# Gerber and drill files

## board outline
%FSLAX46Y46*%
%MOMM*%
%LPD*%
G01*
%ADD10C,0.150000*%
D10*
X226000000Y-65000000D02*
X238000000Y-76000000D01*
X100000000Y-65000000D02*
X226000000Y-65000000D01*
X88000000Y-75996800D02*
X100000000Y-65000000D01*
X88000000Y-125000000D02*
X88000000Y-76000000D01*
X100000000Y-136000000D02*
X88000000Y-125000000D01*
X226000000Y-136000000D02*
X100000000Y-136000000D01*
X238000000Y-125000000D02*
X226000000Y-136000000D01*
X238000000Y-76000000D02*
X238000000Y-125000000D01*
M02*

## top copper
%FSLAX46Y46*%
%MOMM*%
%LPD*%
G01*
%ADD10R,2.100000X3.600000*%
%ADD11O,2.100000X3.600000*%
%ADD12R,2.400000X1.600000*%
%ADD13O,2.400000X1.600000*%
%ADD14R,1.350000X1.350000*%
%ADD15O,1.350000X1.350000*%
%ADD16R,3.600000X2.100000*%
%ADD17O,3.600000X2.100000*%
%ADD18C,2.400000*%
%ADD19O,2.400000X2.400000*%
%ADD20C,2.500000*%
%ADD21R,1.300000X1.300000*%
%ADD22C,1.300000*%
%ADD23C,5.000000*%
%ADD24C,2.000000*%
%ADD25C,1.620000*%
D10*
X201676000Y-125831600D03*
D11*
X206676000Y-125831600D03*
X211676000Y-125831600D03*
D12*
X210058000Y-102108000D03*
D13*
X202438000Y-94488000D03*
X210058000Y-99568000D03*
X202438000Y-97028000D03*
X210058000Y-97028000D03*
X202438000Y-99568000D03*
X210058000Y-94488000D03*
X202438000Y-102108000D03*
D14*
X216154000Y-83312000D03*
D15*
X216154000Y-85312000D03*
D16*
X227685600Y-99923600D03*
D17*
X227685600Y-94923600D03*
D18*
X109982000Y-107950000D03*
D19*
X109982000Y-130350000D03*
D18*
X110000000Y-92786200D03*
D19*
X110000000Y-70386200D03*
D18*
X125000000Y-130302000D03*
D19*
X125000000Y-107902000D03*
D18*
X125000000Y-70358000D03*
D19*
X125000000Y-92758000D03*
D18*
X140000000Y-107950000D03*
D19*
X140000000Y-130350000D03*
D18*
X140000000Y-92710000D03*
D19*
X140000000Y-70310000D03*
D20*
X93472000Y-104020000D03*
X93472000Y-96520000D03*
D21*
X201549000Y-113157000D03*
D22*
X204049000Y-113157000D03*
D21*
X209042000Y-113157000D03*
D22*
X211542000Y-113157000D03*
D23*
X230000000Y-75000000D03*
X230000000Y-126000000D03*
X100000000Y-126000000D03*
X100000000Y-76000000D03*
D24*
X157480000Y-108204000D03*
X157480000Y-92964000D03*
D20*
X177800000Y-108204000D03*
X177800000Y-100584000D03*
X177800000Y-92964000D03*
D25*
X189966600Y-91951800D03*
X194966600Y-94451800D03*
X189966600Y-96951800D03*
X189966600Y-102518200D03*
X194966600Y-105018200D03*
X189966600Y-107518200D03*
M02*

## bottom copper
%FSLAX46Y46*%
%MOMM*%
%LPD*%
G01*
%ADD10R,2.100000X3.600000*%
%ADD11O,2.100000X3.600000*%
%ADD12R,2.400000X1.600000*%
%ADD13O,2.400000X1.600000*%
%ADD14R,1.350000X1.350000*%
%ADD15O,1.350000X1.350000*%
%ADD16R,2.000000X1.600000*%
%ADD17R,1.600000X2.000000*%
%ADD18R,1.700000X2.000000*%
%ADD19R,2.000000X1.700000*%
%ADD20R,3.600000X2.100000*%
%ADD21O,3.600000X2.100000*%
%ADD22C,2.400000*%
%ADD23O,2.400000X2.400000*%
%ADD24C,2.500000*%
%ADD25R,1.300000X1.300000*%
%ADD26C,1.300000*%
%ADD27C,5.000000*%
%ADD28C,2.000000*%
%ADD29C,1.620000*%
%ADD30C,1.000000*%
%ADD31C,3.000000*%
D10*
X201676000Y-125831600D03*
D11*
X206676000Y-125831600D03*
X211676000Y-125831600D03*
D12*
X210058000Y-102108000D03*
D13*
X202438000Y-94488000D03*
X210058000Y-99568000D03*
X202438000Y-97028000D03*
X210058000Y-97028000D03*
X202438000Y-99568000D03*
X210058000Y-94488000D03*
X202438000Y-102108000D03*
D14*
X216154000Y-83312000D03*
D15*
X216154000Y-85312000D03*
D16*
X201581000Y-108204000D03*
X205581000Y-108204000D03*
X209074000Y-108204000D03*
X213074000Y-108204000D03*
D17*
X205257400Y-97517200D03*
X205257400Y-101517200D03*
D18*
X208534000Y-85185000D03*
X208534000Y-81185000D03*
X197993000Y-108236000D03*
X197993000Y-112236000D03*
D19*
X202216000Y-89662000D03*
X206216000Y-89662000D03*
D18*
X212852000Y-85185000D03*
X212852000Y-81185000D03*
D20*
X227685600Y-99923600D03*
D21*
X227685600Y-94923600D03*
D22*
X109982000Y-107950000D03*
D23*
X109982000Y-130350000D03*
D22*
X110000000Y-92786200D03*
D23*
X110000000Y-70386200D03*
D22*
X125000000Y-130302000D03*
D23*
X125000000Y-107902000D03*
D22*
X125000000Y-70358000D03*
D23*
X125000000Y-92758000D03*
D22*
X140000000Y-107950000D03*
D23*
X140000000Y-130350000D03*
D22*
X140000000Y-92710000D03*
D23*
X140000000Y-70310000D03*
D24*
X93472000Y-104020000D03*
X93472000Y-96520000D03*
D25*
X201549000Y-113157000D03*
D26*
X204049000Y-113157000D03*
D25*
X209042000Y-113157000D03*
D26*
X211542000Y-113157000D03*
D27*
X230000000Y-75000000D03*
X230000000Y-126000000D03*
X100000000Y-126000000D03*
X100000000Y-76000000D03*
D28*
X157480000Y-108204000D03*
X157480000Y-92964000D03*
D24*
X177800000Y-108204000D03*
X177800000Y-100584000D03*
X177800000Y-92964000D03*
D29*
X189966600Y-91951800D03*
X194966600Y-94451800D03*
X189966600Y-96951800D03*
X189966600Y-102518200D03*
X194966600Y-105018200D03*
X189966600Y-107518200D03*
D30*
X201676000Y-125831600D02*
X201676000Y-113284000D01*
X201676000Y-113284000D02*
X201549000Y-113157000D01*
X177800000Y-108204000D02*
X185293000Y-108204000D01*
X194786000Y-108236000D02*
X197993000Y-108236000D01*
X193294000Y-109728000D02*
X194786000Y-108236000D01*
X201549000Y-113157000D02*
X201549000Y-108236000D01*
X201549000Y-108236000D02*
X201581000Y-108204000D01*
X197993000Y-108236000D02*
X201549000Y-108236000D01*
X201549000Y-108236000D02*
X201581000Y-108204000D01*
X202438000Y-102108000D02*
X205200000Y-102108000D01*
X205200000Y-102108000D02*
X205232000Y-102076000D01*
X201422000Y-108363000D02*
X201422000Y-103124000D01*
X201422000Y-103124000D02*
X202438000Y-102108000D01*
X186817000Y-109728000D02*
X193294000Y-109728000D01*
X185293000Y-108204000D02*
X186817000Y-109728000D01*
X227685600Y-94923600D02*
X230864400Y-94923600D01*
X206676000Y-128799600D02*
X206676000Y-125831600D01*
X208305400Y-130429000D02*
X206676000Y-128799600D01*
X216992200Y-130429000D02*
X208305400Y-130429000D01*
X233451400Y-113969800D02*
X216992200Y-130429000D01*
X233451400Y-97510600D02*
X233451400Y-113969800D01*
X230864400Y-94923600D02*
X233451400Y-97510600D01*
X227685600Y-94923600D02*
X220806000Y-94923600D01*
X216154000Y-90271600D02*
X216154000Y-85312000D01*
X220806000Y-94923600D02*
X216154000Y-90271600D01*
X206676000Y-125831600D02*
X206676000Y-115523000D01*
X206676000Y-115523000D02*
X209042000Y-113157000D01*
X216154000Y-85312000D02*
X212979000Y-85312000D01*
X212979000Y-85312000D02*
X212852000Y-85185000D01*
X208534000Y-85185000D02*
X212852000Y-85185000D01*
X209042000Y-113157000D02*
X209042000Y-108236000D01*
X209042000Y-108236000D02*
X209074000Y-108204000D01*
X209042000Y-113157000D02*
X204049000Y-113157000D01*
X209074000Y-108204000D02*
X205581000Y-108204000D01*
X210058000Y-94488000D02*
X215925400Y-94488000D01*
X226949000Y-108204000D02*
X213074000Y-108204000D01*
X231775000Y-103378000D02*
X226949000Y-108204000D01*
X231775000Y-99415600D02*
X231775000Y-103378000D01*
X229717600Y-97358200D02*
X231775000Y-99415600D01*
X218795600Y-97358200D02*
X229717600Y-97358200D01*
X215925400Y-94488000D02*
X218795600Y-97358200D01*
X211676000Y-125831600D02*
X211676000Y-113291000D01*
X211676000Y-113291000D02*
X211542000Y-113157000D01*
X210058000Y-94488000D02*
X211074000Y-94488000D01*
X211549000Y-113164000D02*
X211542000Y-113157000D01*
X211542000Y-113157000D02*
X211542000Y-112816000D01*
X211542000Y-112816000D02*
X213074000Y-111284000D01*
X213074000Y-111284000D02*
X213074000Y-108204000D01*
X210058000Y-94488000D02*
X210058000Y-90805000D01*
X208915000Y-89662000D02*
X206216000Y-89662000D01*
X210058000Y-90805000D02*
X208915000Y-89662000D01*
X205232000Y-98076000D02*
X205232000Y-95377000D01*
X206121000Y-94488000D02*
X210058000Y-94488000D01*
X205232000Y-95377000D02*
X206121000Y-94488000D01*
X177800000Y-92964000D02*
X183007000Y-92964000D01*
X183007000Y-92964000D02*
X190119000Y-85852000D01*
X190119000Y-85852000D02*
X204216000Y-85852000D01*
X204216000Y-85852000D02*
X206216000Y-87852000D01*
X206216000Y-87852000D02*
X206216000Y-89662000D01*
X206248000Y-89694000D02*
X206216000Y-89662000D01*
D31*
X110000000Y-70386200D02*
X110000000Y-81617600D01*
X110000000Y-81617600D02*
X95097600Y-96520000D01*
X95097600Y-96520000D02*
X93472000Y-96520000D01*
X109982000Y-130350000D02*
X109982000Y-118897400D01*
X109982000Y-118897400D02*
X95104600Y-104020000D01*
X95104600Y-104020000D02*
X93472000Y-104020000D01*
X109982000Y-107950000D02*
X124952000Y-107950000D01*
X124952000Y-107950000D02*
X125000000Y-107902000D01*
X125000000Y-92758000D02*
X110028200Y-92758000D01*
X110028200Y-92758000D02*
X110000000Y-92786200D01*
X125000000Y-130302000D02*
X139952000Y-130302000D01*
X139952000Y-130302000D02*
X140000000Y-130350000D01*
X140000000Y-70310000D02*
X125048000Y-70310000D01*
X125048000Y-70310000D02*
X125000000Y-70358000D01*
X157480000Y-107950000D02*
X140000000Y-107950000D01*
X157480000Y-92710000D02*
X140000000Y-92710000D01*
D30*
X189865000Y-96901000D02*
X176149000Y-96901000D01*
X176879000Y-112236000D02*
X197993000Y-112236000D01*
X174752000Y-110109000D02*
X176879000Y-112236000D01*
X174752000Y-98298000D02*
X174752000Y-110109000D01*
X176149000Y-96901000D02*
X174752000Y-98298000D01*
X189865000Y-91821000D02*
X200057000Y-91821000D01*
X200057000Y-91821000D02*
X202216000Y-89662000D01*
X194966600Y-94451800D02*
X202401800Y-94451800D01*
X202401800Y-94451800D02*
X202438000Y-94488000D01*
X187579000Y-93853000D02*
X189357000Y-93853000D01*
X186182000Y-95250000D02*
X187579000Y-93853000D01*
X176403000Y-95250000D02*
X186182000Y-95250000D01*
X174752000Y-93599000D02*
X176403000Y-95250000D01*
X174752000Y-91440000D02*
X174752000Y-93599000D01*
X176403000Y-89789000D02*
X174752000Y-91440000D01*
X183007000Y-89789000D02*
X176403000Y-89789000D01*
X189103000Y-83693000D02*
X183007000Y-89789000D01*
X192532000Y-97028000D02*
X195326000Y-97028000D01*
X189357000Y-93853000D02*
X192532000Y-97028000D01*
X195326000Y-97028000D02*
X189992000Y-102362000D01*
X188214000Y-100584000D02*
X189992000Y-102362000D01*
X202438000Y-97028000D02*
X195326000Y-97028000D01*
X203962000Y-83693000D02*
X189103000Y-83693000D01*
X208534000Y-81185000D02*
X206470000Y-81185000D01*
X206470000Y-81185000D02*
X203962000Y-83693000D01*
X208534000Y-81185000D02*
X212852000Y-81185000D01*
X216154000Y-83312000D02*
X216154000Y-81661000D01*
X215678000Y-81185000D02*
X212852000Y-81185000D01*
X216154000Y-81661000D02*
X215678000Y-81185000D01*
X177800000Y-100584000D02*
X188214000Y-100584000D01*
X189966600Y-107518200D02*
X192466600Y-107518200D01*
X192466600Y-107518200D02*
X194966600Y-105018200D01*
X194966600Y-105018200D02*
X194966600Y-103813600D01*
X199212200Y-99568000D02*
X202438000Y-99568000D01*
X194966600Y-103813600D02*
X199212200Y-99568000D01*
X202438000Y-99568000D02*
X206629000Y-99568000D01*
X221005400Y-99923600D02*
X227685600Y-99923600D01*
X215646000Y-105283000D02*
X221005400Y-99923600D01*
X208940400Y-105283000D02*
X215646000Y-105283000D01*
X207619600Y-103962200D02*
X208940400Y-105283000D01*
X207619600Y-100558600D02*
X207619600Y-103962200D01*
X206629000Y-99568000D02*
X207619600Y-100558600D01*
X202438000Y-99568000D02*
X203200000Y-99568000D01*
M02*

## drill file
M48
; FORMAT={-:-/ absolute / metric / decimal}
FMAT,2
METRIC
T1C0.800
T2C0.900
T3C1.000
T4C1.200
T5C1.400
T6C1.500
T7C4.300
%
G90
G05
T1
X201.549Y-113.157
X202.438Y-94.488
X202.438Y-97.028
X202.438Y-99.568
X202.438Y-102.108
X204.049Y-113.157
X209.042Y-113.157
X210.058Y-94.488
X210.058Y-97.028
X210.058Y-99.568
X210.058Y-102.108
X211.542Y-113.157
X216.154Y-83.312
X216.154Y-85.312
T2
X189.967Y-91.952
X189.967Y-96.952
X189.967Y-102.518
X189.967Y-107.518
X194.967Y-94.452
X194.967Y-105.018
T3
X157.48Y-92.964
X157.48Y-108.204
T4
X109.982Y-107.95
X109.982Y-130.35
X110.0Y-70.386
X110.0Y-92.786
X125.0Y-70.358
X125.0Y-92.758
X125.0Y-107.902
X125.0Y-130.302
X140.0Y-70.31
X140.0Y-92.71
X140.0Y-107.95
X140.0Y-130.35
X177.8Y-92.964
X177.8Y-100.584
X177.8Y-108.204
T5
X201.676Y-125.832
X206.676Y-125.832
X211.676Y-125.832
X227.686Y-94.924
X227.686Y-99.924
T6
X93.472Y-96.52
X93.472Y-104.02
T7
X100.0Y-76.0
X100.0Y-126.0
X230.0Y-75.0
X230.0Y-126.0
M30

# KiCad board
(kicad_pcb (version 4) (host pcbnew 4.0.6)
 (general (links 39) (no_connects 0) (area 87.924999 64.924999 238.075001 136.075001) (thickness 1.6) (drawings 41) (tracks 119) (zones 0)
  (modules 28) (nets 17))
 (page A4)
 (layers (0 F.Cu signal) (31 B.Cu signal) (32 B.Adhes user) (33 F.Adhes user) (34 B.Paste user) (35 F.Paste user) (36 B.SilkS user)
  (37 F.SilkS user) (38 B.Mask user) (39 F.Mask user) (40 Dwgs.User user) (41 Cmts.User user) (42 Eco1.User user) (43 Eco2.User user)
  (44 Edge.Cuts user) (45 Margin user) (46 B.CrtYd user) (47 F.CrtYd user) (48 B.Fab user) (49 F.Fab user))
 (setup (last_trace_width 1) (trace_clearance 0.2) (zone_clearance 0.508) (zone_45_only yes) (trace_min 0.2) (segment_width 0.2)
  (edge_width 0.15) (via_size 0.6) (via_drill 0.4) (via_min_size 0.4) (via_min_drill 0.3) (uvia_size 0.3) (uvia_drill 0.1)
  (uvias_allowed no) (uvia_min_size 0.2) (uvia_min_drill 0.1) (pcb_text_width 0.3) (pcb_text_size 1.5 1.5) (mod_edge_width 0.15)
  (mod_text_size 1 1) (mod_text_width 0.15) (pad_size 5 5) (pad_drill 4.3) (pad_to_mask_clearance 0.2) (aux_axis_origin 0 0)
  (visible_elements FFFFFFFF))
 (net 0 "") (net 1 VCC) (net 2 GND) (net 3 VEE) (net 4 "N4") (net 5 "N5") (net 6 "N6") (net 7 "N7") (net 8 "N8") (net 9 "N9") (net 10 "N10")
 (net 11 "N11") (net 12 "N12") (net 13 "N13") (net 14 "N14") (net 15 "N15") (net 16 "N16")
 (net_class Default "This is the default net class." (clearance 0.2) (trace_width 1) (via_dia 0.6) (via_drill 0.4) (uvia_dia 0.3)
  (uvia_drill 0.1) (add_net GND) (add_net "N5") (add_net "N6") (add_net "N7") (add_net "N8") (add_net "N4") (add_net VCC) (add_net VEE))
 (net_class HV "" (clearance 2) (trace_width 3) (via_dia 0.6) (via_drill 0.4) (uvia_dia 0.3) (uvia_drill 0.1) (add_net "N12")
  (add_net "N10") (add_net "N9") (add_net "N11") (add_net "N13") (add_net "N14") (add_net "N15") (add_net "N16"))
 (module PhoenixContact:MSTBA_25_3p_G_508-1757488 (layer F.Cu) (at 201.676 125.8316)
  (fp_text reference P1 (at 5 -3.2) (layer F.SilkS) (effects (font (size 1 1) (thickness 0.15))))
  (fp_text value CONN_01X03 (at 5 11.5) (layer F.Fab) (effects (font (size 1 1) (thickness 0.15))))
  (pad 1 thru_hole rect (at 0 0) (size 2.1 3.6) (drill 1.4) (layers *.Cu *.Mask) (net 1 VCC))
  (pad 2 thru_hole oval (at 5 0) (size 2.1 3.6) (drill 1.4) (layers *.Cu *.Mask) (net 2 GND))
  (pad 3 thru_hole oval (at 10 0) (size 2.1 3.6) (drill 1.4) (layers *.Cu *.Mask) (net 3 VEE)))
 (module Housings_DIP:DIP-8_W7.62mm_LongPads (layer F.Cu) (at 210.058 102.108 180)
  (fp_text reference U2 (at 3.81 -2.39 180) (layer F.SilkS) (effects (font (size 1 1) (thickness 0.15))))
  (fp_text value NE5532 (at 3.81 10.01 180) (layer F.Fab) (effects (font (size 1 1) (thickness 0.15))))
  (pad 1 thru_hole rect (at 0 0 180) (size 2.4 1.6) (drill 0.8) (layers *.Cu *.Mask))
  (pad 5 thru_hole oval (at 7.62 7.62 180) (size 2.4 1.6) (drill 0.8) (layers *.Cu *.Mask) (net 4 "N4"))
  (pad 2 thru_hole oval (at 0 2.54 180) (size 2.4 1.6) (drill 0.8) (layers *.Cu *.Mask))
  (pad 6 thru_hole oval (at 7.62 5.08 180) (size 2.4 1.6) (drill 0.8) (layers *.Cu *.Mask) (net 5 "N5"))
  (pad 3 thru_hole oval (at 0 5.08 180) (size 2.4 1.6) (drill 0.8) (layers *.Cu *.Mask))
  (pad 7 thru_hole oval (at 7.62 2.54 180) (size 2.4 1.6) (drill 0.8) (layers *.Cu *.Mask) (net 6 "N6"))
  (pad 4 thru_hole oval (at 0 7.62 180) (size 2.4 1.6) (drill 0.8) (layers *.Cu *.Mask) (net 3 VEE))
  (pad 8 thru_hole oval (at 7.62 0 180) (size 2.4 1.6) (drill 0.8) (layers *.Cu *.Mask) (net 1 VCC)))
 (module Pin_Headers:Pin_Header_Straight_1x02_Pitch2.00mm (layer F.Cu) (at 216.154 83.312)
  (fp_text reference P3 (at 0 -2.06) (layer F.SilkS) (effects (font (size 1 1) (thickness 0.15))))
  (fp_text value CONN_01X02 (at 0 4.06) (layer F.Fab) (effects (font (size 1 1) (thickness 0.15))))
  (pad 1 thru_hole rect (at 0 0) (size 1.35 1.35) (drill 0.8) (layers *.Cu *.Mask) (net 5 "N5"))
  (pad 2 thru_hole oval (at 0 2) (size 1.35 1.35) (drill 0.8) (layers *.Cu *.Mask) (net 2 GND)))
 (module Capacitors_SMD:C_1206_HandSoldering (layer B.Cu) (at 203.581 108.204)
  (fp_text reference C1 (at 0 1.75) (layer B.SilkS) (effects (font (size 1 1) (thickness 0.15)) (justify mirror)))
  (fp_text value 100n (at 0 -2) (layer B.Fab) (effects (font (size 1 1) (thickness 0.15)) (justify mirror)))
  (pad 1 smd rect (at -2 0) (size 2 1.6) (layers B.Cu B.Paste B.Mask) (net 1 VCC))
  (pad 2 smd rect (at 2 0) (size 2 1.6) (layers B.Cu B.Paste B.Mask) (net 2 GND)))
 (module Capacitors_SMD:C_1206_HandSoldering (layer B.Cu) (at 211.074 108.204)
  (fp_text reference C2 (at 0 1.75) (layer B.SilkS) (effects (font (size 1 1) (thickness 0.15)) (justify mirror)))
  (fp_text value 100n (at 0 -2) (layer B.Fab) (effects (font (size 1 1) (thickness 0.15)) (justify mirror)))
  (pad 1 smd rect (at -2 0) (size 2 1.6) (layers B.Cu B.Paste B.Mask) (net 2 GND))
  (pad 2 smd rect (at 2 0) (size 2 1.6) (layers B.Cu B.Paste B.Mask) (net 3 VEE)))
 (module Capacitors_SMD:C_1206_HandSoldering (layer B.Cu) (at 205.2574 99.5172 270)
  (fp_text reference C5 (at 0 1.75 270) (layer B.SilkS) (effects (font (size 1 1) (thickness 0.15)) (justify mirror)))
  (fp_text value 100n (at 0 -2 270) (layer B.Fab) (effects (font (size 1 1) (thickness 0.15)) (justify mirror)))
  (pad 1 smd rect (at -2 0 270) (size 2 1.6) (layers B.Cu B.Paste B.Mask) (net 3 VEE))
  (pad 2 smd rect (at 2 0 270) (size 2 1.6) (layers B.Cu B.Paste B.Mask) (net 1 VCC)))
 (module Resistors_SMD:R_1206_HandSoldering (layer B.Cu) (at 208.534 83.185 90)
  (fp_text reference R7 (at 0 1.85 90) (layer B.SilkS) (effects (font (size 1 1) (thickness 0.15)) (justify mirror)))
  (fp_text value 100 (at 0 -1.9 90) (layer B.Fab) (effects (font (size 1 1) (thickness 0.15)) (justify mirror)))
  (pad 1 smd rect (at -2 0 90) (size 2 1.7) (layers B.Cu B.Paste B.Mask) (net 2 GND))
  (pad 2 smd rect (at 2 0 90) (size 2 1.7) (layers B.Cu B.Paste B.Mask) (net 5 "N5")))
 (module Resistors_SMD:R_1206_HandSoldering (layer B.Cu) (at 197.993 110.236 270)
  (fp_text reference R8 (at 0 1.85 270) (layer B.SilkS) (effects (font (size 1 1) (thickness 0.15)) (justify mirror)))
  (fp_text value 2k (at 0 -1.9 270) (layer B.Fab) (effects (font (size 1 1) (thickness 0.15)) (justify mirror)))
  (pad 1 smd rect (at -2 0 270) (size 2 1.7) (layers B.Cu B.Paste B.Mask) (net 1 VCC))
  (pad 2 smd rect (at 2 0 270) (size 2 1.7) (layers B.Cu B.Paste B.Mask) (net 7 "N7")))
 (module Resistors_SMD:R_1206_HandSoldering (layer B.Cu) (at 204.216 89.662)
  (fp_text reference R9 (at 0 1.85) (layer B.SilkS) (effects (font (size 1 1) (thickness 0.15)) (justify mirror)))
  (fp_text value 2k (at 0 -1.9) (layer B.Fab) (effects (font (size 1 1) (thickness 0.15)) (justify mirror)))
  (pad 1 smd rect (at -2 0) (size 2 1.7) (layers B.Cu B.Paste B.Mask) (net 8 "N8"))
  (pad 2 smd rect (at 2 0) (size 2 1.7) (layers B.Cu B.Paste B.Mask) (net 3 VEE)))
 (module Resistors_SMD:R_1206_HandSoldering (layer B.Cu) (at 212.852 83.185 90)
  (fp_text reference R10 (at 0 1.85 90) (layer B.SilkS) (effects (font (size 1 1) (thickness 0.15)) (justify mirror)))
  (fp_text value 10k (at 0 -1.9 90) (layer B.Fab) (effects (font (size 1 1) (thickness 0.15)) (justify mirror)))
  (pad 1 smd rect (at -2 0 90) (size 2 1.7) (layers B.Cu B.Paste B.Mask) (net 2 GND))
  (pad 2 smd rect (at 2 0 90) (size 2 1.7) (layers B.Cu B.Paste B.Mask) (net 5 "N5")))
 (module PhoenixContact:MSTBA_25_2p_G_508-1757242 (layer F.Cu) (at 227.6856 99.9236 90)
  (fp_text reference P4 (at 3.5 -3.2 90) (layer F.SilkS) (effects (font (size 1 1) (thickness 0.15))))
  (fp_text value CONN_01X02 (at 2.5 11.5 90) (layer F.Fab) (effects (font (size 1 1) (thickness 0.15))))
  (pad 1 thru_hole rect (at 0 0 90) (size 2.1 3.6) (drill 1.4) (layers *.Cu *.Mask) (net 6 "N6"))
  (pad 2 thru_hole oval (at 5 0 90) (size 2.1 3.6) (drill 1.4) (layers *.Cu *.Mask) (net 2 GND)))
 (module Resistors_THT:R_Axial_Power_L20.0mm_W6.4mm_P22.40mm (layer F.Cu) (at 109.982 107.95 270)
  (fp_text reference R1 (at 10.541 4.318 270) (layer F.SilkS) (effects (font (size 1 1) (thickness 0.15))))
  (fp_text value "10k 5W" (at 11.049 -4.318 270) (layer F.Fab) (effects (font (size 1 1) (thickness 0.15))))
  (pad 1 thru_hole circle (at 0 0 270) (size 2.4 2.4) (drill 1.2) (layers *.Cu *.Mask) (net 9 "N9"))
  (pad 2 thru_hole oval (at 22.4 0 270) (size 2.4 2.4) (drill 1.2) (layers *.Cu *.Mask) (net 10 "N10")))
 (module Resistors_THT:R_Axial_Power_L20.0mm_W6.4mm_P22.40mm (layer F.Cu) (at 110 92.7862 90)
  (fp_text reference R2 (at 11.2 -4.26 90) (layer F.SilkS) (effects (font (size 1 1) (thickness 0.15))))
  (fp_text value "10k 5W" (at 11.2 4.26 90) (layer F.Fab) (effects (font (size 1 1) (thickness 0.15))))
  (pad 1 thru_hole circle (at 0 0 90) (size 2.4 2.4) (drill 1.2) (layers *.Cu *.Mask) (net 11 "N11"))
  (pad 2 thru_hole oval (at 22.4 0 90) (size 2.4 2.4) (drill 1.2) (layers *.Cu *.Mask) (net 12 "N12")))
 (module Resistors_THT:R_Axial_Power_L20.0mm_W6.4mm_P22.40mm (layer F.Cu) (at 125 130.302 90)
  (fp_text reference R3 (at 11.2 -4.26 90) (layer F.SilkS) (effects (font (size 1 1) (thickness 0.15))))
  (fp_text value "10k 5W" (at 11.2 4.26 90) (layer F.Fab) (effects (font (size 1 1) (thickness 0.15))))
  (pad 1 thru_hole circle (at 0 0 90) (size 2.4 2.4) (drill 1.2) (layers *.Cu *.Mask) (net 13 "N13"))
  (pad 2 thru_hole oval (at 22.4 0 90) (size 2.4 2.4) (drill 1.2) (layers *.Cu *.Mask) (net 9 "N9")))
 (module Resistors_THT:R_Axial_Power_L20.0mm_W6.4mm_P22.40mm (layer F.Cu) (at 125 70.358 270)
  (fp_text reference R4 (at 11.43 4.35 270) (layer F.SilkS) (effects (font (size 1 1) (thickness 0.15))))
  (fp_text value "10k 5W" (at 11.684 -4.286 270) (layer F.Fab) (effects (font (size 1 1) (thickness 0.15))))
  (pad 1 thru_hole circle (at 0 0 270) (size 2.4 2.4) (drill 1.2) (layers *.Cu *.Mask) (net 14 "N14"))
  (pad 2 thru_hole oval (at 22.4 0 270) (size 2.4 2.4) (drill 1.2) (layers *.Cu *.Mask) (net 11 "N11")))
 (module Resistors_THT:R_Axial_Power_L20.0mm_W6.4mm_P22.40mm (layer F.Cu) (at 140 107.95 270)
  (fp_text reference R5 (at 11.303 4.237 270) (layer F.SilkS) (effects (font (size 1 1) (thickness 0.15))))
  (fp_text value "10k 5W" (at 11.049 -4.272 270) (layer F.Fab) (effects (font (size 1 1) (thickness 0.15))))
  (pad 1 thru_hole circle (at 0 0 270) (size 2.4 2.4) (drill 1.2) (layers *.Cu *.Mask) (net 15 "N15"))
  (pad 2 thru_hole oval (at 22.4 0 270) (size 2.4 2.4) (drill 1.2) (layers *.Cu *.Mask) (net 13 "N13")))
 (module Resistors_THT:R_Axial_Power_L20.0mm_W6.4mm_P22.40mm (layer F.Cu) (at 140 92.71 90)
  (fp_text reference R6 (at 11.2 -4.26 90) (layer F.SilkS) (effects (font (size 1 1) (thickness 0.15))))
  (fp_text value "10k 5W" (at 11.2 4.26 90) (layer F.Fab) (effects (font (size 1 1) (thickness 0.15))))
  (pad 1 thru_hole circle (at 0 0 90) (size 2.4 2.4) (drill 1.2) (layers *.Cu *.Mask) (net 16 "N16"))
  (pad 2 thru_hole oval (at 22.4 0 90) (size 2.4 2.4) (drill 1.2) (layers *.Cu *.Mask) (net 14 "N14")))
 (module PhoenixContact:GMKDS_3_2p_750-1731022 (layer F.Cu) (at 93.472 96.52 270)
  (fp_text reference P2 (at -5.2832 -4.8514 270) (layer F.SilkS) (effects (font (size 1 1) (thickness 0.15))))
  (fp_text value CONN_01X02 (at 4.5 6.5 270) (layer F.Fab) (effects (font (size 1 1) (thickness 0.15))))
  (pad 2 thru_hole circle (at 7.5 0 270) (size 2.5 2.5) (drill 1.5) (layers *.Cu *.Mask) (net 10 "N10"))
  (pad 1 thru_hole circle (at 0 0 270) (size 2.5 2.5) (drill 1.5) (layers *.Cu *.Mask) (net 12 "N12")))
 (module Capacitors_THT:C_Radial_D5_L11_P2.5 (layer F.Cu) (at 201.549 113.157)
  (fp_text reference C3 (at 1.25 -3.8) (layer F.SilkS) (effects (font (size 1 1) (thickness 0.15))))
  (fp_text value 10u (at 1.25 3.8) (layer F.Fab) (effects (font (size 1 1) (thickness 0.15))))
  (pad 1 thru_hole rect (at 0 0) (size 1.3 1.3) (drill 0.8) (layers *.Cu *.Mask) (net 1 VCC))
  (pad 2 thru_hole circle (at 2.5 0) (size 1.3 1.3) (drill 0.8) (layers *.Cu *.Mask) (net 2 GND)))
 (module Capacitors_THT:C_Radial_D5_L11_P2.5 (layer F.Cu) (at 209.042 113.157)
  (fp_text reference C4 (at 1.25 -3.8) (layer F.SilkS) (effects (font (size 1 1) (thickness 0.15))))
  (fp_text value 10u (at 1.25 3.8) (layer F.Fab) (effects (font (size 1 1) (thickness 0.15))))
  (pad 1 thru_hole rect (at 0 0) (size 1.3 1.3) (drill 0.8) (layers *.Cu *.Mask) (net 2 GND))
  (pad 2 thru_hole circle (at 2.5 0) (size 1.3 1.3) (drill 0.8) (layers *.Cu *.Mask) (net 3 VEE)))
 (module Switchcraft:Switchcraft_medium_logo (layer F.Cu) (at 208.7372 69.3166)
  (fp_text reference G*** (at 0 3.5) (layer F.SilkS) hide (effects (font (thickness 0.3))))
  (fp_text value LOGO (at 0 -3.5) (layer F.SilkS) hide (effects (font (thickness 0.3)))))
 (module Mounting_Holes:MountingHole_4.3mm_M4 (layer F.Cu) (at 230 75)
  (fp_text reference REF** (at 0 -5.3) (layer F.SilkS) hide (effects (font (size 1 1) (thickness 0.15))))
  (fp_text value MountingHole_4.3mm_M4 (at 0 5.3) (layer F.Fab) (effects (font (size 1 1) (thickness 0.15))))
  (pad "" np_thru_hole circle (at 0 0) (size 5 5) (drill 4.3) (layers *.Cu *.Mask)))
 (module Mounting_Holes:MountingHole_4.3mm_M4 (layer F.Cu) (at 230 126)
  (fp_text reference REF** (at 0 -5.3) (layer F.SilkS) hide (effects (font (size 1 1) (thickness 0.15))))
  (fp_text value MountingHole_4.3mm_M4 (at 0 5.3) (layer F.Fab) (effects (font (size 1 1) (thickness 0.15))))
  (pad "" np_thru_hole circle (at 0 0) (size 5 5) (drill 4.3) (layers *.Cu *.Mask)))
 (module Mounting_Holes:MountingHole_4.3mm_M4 (layer F.Cu) (at 100 126)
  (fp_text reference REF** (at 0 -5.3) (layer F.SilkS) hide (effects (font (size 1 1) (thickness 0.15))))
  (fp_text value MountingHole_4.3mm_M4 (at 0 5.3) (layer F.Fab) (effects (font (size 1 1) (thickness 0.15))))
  (pad "" np_thru_hole circle (at 0 0) (size 5 5) (drill 4.3) (layers *.Cu *.Mask)))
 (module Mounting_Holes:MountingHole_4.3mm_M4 (layer F.Cu) (at 100 76)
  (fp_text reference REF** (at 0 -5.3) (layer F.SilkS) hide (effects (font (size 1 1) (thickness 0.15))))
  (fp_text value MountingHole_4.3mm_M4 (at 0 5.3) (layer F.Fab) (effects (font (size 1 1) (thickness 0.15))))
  (pad "" np_thru_hole circle (at 0 0) (size 5 5) (drill 4.3) (layers *.Cu *.Mask)))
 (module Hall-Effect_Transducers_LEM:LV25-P (layer F.Cu) (at 167.64 100.584 90)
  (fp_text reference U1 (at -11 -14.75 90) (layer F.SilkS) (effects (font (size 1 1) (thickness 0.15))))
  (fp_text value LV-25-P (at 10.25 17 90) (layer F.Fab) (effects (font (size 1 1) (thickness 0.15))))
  (pad 1 thru_hole circle (at -7.62 -10.16 90) (size 2 2) (drill 1) (layers *.Cu *.Mask) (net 15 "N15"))
  (pad 2 thru_hole circle (at 7.62 -10.16 90) (size 2 2) (drill 1) (layers *.Cu *.Mask) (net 16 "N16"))
  (pad 3 thru_hole circle (at -7.62 10.16 90) (size 2.5 2.5) (drill 1.2) (layers *.Cu *.Mask) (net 1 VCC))
  (pad 4 thru_hole circle (at 0 10.16 90) (size 2.5 2.5) (drill 1.2) (layers *.Cu *.Mask) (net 5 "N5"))
  (pad 5 thru_hole circle (at 7.62 10.16 90) (size 2.5 2.5) (drill 1.2) (layers *.Cu *.Mask) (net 3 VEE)))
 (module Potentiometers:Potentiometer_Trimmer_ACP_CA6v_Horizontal (layer F.Cu) (at 189.9666 96.9518)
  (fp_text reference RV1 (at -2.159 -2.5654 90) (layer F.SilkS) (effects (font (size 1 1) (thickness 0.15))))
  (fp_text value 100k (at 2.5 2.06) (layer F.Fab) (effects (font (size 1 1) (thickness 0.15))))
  (pad 3 thru_hole circle (at 0 -5) (size 1.62 1.62) (drill 0.9) (layers *.Cu *.Mask) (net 8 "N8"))
  (pad 2 thru_hole circle (at 5 -2.5) (size 1.62 1.62) (drill 0.9) (layers *.Cu *.Mask) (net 4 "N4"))
  (pad 1 thru_hole circle (at 0 0) (size 1.62 1.62) (drill 0.9) (layers *.Cu *.Mask) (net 7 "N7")))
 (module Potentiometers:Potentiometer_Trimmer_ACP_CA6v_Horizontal (layer F.Cu) (at 189.9666 107.5182)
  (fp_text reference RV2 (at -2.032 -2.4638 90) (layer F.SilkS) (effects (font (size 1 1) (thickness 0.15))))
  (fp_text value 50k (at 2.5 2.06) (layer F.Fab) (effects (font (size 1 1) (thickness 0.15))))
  (pad 3 thru_hole circle (at 0 -5) (size 1.62 1.62) (drill 0.9) (layers *.Cu *.Mask) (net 5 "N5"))
  (pad 2 thru_hole circle (at 5 -2.5) (size 1.62 1.62) (drill 0.9) (layers *.Cu *.Mask) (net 6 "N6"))
  (pad 1 thru_hole circle (at 0 0) (size 1.62 1.62) (drill 0.9) (layers *.Cu *.Mask) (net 6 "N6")))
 (gr_line (start 226 65) (end 238 76) (angle 90) (layer Edge.Cuts) (width 0.15))
 (gr_line (start 100 65) (end 226 65) (angle 90) (layer Edge.Cuts) (width 0.15))
 (gr_line (start 88 75.9968) (end 100 65) (angle 90) (layer Edge.Cuts) (width 0.15))
 (gr_line (start 88 125) (end 88 76) (angle 90) (layer Edge.Cuts) (width 0.15))
 (gr_line (start 100 136) (end 88 125) (angle 90) (layer Edge.Cuts) (width 0.15))
 (gr_line (start 226 136) (end 100 136) (angle 90) (layer Edge.Cuts) (width 0.15))
 (gr_line (start 238 125) (end 226 136) (angle 90) (layer Edge.Cuts) (width 0.15))
 (gr_line (start 238 76) (end 238 125) (angle 90) (layer Edge.Cuts) (width 0.15))
 (segment (start 201.676 125.8316) (end 201.676 113.284) (width 1) (layer B.Cu) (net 1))
 (segment (start 201.676 113.284) (end 201.549 113.157) (width 1) (layer B.Cu) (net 1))
 (segment (start 177.8 108.204) (end 185.293 108.204) (width 1) (layer B.Cu) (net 1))
 (segment (start 194.786 108.236) (end 197.993 108.236) (width 1) (layer B.Cu) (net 1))
 (segment (start 193.294 109.728) (end 194.786 108.236) (width 1) (layer B.Cu) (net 1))
 (segment (start 201.549 113.157) (end 201.549 108.236) (width 1) (layer B.Cu) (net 1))
 (segment (start 201.549 108.236) (end 201.581 108.204) (width 1) (layer B.Cu) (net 1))
 (segment (start 197.993 108.236) (end 201.549 108.236) (width 1) (layer B.Cu) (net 1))
 (segment (start 201.549 108.236) (end 201.581 108.204) (width 1) (layer B.Cu) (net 1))
 (segment (start 202.438 102.108) (end 205.2 102.108) (width 1) (layer B.Cu) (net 1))
 (segment (start 205.2 102.108) (end 205.232 102.076) (width 1) (layer B.Cu) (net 1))
 (segment (start 201.422 108.363) (end 201.422 103.124) (width 1) (layer B.Cu) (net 1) (status 10))
 (segment (start 201.422 103.124) (end 202.438 102.108) (width 1) (layer B.Cu) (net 1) (status 20))
 (segment (start 186.817 109.728) (end 193.294 109.728) (width 1) (layer B.Cu) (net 1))
 (segment (start 185.293 108.204) (end 186.817 109.728) (width 1) (layer B.Cu) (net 1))
 (segment (start 227.6856 94.9236) (end 230.8644 94.9236) (width 1) (layer B.Cu) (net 2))
 (segment (start 206.676 128.7996) (end 206.676 125.8316) (width 1) (layer B.Cu) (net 2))
 (segment (start 208.3054 130.429) (end 206.676 128.7996) (width 1) (layer B.Cu) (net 2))
 (segment (start 216.9922 130.429) (end 208.3054 130.429) (width 1) (layer B.Cu) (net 2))
 (segment (start 233.4514 113.9698) (end 216.9922 130.429) (width 1) (layer B.Cu) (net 2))
 (segment (start 233.4514 97.5106) (end 233.4514 113.9698) (width 1) (layer B.Cu) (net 2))
 (segment (start 230.8644 94.9236) (end 233.4514 97.5106) (width 1) (layer B.Cu) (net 2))
 (segment (start 227.6856 94.9236) (end 220.806 94.9236) (width 1) (layer B.Cu) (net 2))
 (segment (start 216.154 90.2716) (end 216.154 85.312) (width 1) (layer B.Cu) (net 2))
 (segment (start 220.806 94.9236) (end 216.154 90.2716) (width 1) (layer B.Cu) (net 2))
 (segment (start 206.676 125.8316) (end 206.676 115.523) (width 1) (layer B.Cu) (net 2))
 (segment (start 206.676 115.523) (end 209.042 113.157) (width 1) (layer B.Cu) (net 2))
 (segment (start 216.154 85.312) (end 212.979 85.312) (width 1) (layer B.Cu) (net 2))
 (segment (start 212.979 85.312) (end 212.852 85.185) (width 1) (layer B.Cu) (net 2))
 (segment (start 208.534 85.185) (end 212.852 85.185) (width 1) (layer B.Cu) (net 2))
 (segment (start 209.042 113.157) (end 209.042 108.236) (width 1) (layer B.Cu) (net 2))
 (segment (start 209.042 108.236) (end 209.074 108.204) (width 1) (layer B.Cu) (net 2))
 (segment (start 209.042 113.157) (end 204.049 113.157) (width 1) (layer B.Cu) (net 2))
 (segment (start 209.074 108.204) (end 205.581 108.204) (width 1) (layer B.Cu) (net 2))
 (segment (start 210.058 94.488) (end 215.9254 94.488) (width 1) (layer B.Cu) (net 3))
 (segment (start 226.949 108.204) (end 213.074 108.204) (width 1) (layer B.Cu) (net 3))
 (segment (start 231.775 103.378) (end 226.949 108.204) (width 1) (layer B.Cu) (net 3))
 (segment (start 231.775 99.4156) (end 231.775 103.378) (width 1) (layer B.Cu) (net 3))
 (segment (start 229.7176 97.3582) (end 231.775 99.4156) (width 1) (layer B.Cu) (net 3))
 (segment (start 218.7956 97.3582) (end 229.7176 97.3582) (width 1) (layer B.Cu) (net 3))
 (segment (start 215.9254 94.488) (end 218.7956 97.3582) (width 1) (layer B.Cu) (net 3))
 (segment (start 211.676 125.8316) (end 211.676 113.291) (width 1) (layer B.Cu) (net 3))
 (segment (start 211.676 113.291) (end 211.542 113.157) (width 1) (layer B.Cu) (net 3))
 (segment (start 210.058 94.488) (end 211.074 94.488) (width 1) (layer B.Cu) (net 3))
 (segment (start 211.549 113.164) (end 211.542 113.157) (width 1) (layer B.Cu) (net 3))
 (segment (start 211.542 113.157) (end 211.542 112.816) (width 1) (layer B.Cu) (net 3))
 (segment (start 211.542 112.816) (end 213.074 111.284) (width 1) (layer B.Cu) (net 3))
 (segment (start 213.074 111.284) (end 213.074 108.204) (width 1) (layer B.Cu) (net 3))
 (segment (start 210.058 94.488) (end 210.058 90.805) (width 1) (layer B.Cu) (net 3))
 (segment (start 208.915 89.662) (end 206.216 89.662) (width 1) (layer B.Cu) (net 3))
 (segment (start 210.058 90.805) (end 208.915 89.662) (width 1) (layer B.Cu) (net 3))
 (segment (start 205.232 98.076) (end 205.232 95.377) (width 1) (layer B.Cu) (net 3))
 (segment (start 206.121 94.488) (end 210.058 94.488) (width 1) (layer B.Cu) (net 3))
 (segment (start 205.232 95.377) (end 206.121 94.488) (width 1) (layer B.Cu) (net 3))
 (segment (start 177.8 92.964) (end 183.007 92.964) (width 1) (layer B.Cu) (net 3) (status 10))
 (segment (start 183.007 92.964) (end 190.119 85.852) (width 1) (layer B.Cu) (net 3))
 (segment (start 190.119 85.852) (end 204.216 85.852) (width 1) (layer B.Cu) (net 3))
 (segment (start 204.216 85.852) (end 206.216 87.852) (width 1) (layer B.Cu) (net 3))
 (segment (start 206.216 87.852) (end 206.216 89.662) (width 1) (layer B.Cu) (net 3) (status 20))
 (segment (start 206.248 89.694) (end 206.216 89.662) (width 1) (layer B.Cu) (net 3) (status 30))
 (segment (start 110 70.3862) (end 110 81.6176) (width 3) (layer B.Cu) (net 12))
 (segment (start 110 81.6176) (end 95.0976 96.52) (width 3) (layer B.Cu) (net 12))
 (segment (start 95.0976 96.52) (end 93.472 96.52) (width 3) (layer B.Cu) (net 12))
 (segment (start 109.982 130.35) (end 109.982 118.8974) (width 3) (layer B.Cu) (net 10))
 (segment (start 109.982 118.8974) (end 95.1046 104.02) (width 3) (layer B.Cu) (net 10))
 (segment (start 95.1046 104.02) (end 93.472 104.02) (width 3) (layer B.Cu) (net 10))
 (segment (start 109.982 107.95) (end 124.952 107.95) (width 3) (layer B.Cu) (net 9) (status 30))
 (segment (start 124.952 107.95) (end 125 107.902) (width 3) (layer B.Cu) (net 9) (status 30))
 (segment (start 125 92.758) (end 110.0282 92.758) (width 3) (layer B.Cu) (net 11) (status 30))
 (segment (start 110.0282 92.758) (end 110 92.7862) (width 3) (layer B.Cu) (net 11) (status 30))
 (segment (start 125 130.302) (end 139.952 130.302) (width 3) (layer B.Cu) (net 13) (status 30))
 (segment (start 139.952 130.302) (end 140 130.35) (width 3) (layer B.Cu) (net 13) (status 30))
 (segment (start 140 70.31) (end 125.048 70.31) (width 3) (layer B.Cu) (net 14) (status 30))
 (segment (start 125.048 70.31) (end 125 70.358) (width 3) (layer B.Cu) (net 14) (status 30))
 (segment (start 157.48 107.95) (end 140 107.95) (width 3) (layer B.Cu) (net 15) (status 30))
 (segment (start 157.48 92.71) (end 140 92.71) (width 3) (layer B.Cu) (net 16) (status 30))
 (segment (start 189.865 96.901) (end 176.149 96.901) (width 1) (layer B.Cu) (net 7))
 (segment (start 176.879 112.236) (end 197.993 112.236) (width 1) (layer B.Cu) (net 7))
 (segment (start 174.752 110.109) (end 176.879 112.236) (width 1) (layer B.Cu) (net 7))
 (segment (start 174.752 98.298) (end 174.752 110.109) (width 1) (layer B.Cu) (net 7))
 (segment (start 176.149 96.901) (end 174.752 98.298) (width 1) (layer B.Cu) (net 7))
 (segment (start 189.865 91.821) (end 200.057 91.821) (width 1) (layer B.Cu) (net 8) (status 10))
 (segment (start 200.057 91.821) (end 202.216 89.662) (width 1) (layer B.Cu) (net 8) (status 20))
 (segment (start 194.9666 94.4518) (end 202.4018 94.4518) (width 1) (layer B.Cu) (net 4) (status C00000))
 (segment (start 202.4018 94.4518) (end 202.438 94.488) (width 1) (layer B.Cu) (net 4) (status C00000))
 (segment (start 187.579 93.853) (end 189.357 93.853) (width 1) (layer B.Cu) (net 5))
 (segment (start 186.182 95.25) (end 187.579 93.853) (width 1) (layer B.Cu) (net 5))
 (segment (start 176.403 95.25) (end 186.182 95.25) (width 1) (layer B.Cu) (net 5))
 (segment (start 174.752 93.599) (end 176.403 95.25) (width 1) (layer B.Cu) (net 5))
 (segment (start 174.752 91.44) (end 174.752 93.599) (width 1) (layer B.Cu) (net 5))
 (segment (start 176.403 89.789) (end 174.752 91.44) (width 1) (layer B.Cu) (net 5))
 (segment (start 183.007 89.789) (end 176.403 89.789) (width 1) (layer B.Cu) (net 5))
 (segment (start 189.103 83.693) (end 183.007 89.789) (width 1) (layer B.Cu) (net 5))
 (segment (start 192.532 97.028) (end 195.326 97.028) (width 1) (layer B.Cu) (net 5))
 (segment (start 189.357 93.853) (end 192.532 97.028) (width 1) (layer B.Cu) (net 5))
 (segment (start 195.326 97.028) (end 189.992 102.362) (width 1) (layer B.Cu) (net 5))
 (segment (start 188.214 100.584) (end 189.992 102.362) (width 1) (layer B.Cu) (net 5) (status 20))
 (segment (start 202.438 97.028) (end 195.326 97.028) (width 1) (layer B.Cu) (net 5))
 (segment (start 203.962 83.693) (end 189.103 83.693) (width 1) (layer B.Cu) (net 5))
 (segment (start 208.534 81.185) (end 206.47 81.185) (width 1) (layer B.Cu) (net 5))
 (segment (start 206.47 81.185) (end 203.962 83.693) (width 1) (layer B.Cu) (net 5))
 (segment (start 208.534 81.185) (end 212.852 81.185) (width 1) (layer B.Cu) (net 5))
 (segment (start 216.154 83.312) (end 216.154 81.661) (width 1) (layer B.Cu) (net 5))
 (segment (start 215.678 81.185) (end 212.852 81.185) (width 1) (layer B.Cu) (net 5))
 (segment (start 216.154 81.661) (end 215.678 81.185) (width 1) (layer B.Cu) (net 5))
 (segment (start 177.8 100.584) (end 188.214 100.584) (width 1) (layer B.Cu) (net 5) (status 10))
 (segment (start 189.9666 107.5182) (end 192.4666 107.5182) (width 1) (layer B.Cu) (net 6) (status 400000))
 (segment (start 192.4666 107.5182) (end 194.9666 105.0182) (width 1) (layer B.Cu) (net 6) (status 800000))
 (segment (start 194.9666 105.0182) (end 194.9666 103.8136) (width 1) (layer B.Cu) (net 6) (status 400000))
 (segment (start 199.2122 99.568) (end 202.438 99.568) (width 1) (layer B.Cu) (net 6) (status 800000))
 (segment (start 194.9666 103.8136) (end 199.2122 99.568) (width 1) (layer B.Cu) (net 6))
 (segment (start 202.438 99.568) (end 206.629 99.568) (width 1) (layer B.Cu) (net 6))
 (segment (start 221.0054 99.9236) (end 227.6856 99.9236) (width 1) (layer B.Cu) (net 6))
 (segment (start 215.646 105.283) (end 221.0054 99.9236) (width 1) (layer B.Cu) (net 6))
 (segment (start 208.9404 105.283) (end 215.646 105.283) (width 1) (layer B.Cu) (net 6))
 (segment (start 207.6196 103.9622) (end 208.9404 105.283) (width 1) (layer B.Cu) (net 6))
 (segment (start 207.6196 100.5586) (end 207.6196 103.9622) (width 1) (layer B.Cu) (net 6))
 (segment (start 206.629 99.568) (end 207.6196 100.5586) (width 1) (layer B.Cu) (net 6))
 (segment (start 202.438 99.568) (end 203.2 99.568) (width 1) (layer B.Cu) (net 6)))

